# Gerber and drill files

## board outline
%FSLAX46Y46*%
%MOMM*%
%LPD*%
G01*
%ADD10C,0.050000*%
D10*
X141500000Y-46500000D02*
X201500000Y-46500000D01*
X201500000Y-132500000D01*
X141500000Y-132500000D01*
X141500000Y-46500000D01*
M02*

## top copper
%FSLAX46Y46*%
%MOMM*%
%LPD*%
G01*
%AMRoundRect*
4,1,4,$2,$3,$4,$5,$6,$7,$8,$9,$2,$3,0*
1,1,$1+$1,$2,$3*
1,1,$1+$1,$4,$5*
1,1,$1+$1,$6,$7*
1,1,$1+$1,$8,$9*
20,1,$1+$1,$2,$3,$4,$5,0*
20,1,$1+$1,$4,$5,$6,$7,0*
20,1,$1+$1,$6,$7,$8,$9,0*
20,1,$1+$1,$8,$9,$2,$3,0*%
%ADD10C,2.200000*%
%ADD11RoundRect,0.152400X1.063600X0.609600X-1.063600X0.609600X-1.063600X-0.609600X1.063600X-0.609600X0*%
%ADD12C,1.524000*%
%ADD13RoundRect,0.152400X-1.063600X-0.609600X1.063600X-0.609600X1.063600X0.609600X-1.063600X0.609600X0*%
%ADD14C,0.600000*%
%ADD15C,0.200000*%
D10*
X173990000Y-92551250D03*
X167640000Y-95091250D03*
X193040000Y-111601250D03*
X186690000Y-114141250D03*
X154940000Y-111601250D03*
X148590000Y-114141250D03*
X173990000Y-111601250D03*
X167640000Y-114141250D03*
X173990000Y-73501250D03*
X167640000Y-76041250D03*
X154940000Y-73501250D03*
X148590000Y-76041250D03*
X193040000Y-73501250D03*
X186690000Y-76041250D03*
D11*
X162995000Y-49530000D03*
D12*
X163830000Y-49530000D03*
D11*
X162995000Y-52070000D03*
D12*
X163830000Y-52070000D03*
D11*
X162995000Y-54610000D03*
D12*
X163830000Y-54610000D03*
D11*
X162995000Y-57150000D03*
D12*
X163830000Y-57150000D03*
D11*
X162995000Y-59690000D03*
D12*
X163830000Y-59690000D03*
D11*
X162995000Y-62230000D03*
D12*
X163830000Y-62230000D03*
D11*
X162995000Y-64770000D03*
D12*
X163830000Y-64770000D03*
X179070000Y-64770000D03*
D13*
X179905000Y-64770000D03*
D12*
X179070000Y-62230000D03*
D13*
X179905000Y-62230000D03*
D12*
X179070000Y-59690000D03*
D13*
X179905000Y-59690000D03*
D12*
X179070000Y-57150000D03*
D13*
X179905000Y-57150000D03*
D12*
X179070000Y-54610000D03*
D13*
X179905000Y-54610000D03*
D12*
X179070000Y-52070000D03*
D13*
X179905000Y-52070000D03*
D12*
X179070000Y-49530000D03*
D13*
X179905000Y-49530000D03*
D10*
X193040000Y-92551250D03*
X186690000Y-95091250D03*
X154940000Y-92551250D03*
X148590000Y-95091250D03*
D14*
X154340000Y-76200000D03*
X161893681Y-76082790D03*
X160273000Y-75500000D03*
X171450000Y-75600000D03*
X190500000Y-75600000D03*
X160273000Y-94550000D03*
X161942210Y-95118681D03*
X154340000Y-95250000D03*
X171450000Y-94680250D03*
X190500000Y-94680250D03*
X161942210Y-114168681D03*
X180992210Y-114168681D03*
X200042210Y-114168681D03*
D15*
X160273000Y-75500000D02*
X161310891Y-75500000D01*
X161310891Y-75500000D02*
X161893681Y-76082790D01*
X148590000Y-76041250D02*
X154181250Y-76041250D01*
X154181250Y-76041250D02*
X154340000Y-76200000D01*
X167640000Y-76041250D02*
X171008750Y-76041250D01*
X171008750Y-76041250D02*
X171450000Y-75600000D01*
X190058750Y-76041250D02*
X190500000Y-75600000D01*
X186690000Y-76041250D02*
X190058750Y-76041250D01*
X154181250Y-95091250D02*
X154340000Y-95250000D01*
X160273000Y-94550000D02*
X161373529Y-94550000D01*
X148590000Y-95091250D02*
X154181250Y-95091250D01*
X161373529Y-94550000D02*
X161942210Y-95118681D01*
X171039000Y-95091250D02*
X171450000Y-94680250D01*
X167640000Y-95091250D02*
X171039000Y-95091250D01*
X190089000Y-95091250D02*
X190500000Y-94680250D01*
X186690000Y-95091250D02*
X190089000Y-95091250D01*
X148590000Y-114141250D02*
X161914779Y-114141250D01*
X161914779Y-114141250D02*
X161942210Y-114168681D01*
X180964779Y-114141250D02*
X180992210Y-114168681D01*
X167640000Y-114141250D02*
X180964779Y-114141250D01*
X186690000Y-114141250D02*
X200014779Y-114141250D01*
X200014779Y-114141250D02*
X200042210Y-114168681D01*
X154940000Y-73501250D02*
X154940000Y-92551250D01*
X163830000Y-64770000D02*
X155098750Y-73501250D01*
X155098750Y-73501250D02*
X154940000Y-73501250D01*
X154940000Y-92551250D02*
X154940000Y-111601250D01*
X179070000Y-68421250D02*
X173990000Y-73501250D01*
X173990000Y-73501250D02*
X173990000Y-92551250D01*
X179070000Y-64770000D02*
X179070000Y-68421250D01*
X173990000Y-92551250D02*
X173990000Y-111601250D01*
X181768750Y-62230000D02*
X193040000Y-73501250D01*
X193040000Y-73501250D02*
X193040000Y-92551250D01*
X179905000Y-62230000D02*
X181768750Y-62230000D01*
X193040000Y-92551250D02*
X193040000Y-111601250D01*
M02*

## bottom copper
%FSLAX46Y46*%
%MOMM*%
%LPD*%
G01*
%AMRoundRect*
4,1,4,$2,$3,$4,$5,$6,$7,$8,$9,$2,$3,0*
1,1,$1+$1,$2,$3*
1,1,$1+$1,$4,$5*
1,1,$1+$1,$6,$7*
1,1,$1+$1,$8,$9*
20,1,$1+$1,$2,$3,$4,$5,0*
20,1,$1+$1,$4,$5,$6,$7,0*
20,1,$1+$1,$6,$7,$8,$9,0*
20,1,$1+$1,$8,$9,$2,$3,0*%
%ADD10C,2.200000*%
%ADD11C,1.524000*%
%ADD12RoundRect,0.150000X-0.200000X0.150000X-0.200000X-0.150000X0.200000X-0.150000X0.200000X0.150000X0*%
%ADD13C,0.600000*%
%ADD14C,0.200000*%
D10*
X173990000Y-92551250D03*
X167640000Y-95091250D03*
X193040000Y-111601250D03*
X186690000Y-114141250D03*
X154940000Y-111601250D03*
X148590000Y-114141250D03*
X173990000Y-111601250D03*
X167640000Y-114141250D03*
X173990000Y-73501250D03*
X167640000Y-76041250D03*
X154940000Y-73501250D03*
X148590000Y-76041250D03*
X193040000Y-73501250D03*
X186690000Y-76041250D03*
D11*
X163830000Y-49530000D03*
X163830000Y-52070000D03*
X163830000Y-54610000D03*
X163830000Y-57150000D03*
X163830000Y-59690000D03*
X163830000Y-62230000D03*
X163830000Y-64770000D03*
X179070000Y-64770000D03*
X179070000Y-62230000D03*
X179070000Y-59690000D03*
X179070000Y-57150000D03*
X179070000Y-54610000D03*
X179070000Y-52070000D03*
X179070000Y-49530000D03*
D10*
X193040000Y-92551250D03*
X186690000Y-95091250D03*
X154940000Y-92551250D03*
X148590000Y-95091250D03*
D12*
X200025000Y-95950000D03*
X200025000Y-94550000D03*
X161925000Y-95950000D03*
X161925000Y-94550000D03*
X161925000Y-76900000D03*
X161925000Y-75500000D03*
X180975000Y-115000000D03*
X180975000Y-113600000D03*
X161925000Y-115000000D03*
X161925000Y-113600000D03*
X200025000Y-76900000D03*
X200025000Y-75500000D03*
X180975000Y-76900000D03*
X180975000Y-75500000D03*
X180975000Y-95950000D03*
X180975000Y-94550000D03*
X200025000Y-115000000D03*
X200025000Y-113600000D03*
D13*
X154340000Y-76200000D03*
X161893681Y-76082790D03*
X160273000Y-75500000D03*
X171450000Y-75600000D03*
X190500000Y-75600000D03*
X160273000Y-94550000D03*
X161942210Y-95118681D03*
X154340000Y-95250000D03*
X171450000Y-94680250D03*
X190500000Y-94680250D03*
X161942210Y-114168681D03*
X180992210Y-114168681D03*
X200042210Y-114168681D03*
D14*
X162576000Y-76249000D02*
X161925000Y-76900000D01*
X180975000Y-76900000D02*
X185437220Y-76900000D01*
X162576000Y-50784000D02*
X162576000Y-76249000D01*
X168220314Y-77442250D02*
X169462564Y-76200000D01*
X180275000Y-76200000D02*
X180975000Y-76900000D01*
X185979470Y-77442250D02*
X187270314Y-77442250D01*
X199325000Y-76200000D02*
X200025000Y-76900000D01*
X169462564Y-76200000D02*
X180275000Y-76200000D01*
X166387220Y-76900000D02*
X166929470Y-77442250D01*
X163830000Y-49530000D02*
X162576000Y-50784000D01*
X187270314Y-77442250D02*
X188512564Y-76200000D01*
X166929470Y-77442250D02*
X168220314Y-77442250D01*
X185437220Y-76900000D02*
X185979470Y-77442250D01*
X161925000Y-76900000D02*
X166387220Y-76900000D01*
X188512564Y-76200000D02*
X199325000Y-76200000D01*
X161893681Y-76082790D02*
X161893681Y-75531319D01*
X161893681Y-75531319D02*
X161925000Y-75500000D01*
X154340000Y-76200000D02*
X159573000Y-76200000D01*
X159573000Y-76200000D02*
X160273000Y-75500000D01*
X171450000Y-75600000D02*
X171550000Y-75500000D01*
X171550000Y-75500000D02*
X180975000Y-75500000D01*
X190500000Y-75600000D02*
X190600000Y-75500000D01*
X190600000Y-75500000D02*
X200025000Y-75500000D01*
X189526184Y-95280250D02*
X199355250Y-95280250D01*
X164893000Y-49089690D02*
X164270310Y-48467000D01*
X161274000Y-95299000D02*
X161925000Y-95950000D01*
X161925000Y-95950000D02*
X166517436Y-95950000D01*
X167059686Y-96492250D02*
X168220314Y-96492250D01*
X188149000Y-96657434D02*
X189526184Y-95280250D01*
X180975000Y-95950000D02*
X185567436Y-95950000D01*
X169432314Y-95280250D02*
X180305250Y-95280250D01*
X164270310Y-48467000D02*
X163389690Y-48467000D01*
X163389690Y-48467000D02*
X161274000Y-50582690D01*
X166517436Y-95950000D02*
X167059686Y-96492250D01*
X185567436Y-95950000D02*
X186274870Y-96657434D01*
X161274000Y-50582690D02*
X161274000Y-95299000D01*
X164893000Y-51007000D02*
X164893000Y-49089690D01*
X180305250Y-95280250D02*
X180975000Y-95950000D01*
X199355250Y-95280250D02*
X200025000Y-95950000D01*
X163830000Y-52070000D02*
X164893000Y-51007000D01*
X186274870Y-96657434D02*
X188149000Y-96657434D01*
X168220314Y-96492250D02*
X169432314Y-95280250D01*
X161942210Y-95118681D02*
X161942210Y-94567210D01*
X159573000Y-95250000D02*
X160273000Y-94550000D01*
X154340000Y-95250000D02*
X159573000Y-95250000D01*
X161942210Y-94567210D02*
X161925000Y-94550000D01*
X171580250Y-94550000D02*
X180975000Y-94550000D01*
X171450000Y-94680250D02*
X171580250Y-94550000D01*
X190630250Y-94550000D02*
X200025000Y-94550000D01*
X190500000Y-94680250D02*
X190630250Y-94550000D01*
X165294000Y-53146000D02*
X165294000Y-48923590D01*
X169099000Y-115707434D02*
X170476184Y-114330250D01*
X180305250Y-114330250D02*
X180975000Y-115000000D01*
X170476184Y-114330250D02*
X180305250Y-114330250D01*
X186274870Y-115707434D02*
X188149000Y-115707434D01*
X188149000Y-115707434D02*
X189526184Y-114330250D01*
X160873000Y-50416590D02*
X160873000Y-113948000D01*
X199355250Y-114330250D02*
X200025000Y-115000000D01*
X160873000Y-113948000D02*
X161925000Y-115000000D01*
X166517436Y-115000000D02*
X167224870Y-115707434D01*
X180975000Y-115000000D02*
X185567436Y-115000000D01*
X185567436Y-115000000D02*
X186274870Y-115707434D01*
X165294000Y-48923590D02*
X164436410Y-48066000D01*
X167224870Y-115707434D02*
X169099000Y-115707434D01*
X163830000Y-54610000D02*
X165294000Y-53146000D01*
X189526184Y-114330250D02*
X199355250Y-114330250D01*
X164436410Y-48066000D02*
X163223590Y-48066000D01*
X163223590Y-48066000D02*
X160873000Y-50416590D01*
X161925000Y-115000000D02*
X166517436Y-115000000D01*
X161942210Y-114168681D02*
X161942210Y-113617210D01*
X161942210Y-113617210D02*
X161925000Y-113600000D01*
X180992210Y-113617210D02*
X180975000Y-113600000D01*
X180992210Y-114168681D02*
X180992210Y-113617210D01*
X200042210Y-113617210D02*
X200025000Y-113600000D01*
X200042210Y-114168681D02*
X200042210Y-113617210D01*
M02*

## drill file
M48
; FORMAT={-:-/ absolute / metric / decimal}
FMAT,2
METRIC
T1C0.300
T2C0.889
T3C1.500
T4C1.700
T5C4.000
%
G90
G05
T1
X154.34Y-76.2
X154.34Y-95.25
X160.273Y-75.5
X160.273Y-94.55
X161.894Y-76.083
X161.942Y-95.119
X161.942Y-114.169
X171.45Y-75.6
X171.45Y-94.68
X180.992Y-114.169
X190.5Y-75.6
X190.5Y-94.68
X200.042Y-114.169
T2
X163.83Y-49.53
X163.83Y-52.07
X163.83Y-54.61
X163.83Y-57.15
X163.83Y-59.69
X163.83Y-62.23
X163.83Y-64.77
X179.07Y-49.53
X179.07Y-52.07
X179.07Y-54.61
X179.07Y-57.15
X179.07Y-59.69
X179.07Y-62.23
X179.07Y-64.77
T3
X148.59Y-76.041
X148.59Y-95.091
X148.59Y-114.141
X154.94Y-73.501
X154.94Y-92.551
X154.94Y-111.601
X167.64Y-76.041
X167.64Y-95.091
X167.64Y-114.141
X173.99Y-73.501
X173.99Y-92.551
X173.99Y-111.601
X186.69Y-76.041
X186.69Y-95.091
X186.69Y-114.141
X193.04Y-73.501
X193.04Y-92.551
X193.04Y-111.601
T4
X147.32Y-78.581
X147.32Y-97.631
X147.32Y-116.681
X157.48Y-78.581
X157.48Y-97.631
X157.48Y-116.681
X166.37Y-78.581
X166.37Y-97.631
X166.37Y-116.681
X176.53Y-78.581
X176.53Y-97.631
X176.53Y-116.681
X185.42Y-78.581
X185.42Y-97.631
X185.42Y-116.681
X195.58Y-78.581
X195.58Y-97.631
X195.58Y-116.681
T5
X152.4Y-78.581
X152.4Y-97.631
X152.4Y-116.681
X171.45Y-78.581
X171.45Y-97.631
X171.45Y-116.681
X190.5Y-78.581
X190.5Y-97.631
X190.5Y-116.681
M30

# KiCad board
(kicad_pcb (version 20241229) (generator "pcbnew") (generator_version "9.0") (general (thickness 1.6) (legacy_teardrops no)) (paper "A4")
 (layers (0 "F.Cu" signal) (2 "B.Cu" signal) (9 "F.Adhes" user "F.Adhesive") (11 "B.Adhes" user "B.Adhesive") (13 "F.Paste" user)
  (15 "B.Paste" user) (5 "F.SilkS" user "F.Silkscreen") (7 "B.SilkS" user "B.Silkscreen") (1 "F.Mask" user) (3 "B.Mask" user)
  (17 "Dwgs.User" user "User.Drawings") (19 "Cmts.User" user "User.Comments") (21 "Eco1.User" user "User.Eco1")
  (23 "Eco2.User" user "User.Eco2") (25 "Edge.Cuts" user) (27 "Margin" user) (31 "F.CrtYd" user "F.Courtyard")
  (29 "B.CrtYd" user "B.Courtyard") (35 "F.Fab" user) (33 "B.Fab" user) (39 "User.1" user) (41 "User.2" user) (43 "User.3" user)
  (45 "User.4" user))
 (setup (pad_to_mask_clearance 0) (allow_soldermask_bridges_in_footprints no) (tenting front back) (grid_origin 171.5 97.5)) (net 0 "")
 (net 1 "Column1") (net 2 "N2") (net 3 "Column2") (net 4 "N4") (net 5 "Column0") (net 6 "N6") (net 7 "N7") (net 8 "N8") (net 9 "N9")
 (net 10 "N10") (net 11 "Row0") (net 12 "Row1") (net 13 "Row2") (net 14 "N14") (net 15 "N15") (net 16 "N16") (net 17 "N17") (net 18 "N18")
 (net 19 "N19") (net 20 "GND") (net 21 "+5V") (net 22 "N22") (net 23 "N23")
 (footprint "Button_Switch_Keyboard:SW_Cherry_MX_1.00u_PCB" (layer "F.Cu") (at 173.99 92.55125)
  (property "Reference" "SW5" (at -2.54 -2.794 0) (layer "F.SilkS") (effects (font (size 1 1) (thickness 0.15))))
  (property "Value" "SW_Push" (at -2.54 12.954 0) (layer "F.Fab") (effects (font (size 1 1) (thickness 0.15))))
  (pad "" np_thru_hole circle (at -7.62 5.08) (size 1.7 1.7) (drill 1.7) (layers "*.Cu" "*.Mask"))
  (pad "" np_thru_hole circle (at -2.54 5.08) (size 4 4) (drill 4) (layers "*.Cu" "*.Mask"))
  (pad "" np_thru_hole circle (at 2.54 5.08) (size 1.7 1.7) (drill 1.7) (layers "*.Cu" "*.Mask"))
  (pad "1" thru_hole circle (at 0 0) (size 2.2 2.2) (drill 1.5) (layers "*.Cu" "*.Mask") (remove_unused_layers no) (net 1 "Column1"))
  (pad "2" thru_hole circle (at -6.35 2.54) (size 2.2 2.2) (drill 1.5) (layers "*.Cu" "*.Mask") (remove_unused_layers no) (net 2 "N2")))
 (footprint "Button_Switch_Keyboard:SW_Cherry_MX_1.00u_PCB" (layer "F.Cu") (at 193.04 111.60125)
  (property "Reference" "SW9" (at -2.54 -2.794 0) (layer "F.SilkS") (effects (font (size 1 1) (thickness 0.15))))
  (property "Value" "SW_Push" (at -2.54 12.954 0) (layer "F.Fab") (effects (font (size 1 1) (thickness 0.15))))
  (pad "" np_thru_hole circle (at -7.62 5.08) (size 1.7 1.7) (drill 1.7) (layers "*.Cu" "*.Mask"))
  (pad "" np_thru_hole circle (at -2.54 5.08) (size 4 4) (drill 4) (layers "*.Cu" "*.Mask"))
  (pad "" np_thru_hole circle (at 2.54 5.08) (size 1.7 1.7) (drill 1.7) (layers "*.Cu" "*.Mask"))
  (pad "1" thru_hole circle (at 0 0) (size 2.2 2.2) (drill 1.5) (layers "*.Cu" "*.Mask") (remove_unused_layers no) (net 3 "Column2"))
  (pad "2" thru_hole circle (at -6.35 2.54) (size 2.2 2.2) (drill 1.5) (layers "*.Cu" "*.Mask") (remove_unused_layers no) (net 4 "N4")))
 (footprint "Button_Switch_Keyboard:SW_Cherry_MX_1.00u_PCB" (layer "F.Cu") (at 154.94 111.60125)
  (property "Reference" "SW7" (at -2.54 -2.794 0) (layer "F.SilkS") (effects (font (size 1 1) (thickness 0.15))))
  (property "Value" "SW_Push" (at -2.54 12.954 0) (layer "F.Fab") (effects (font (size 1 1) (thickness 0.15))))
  (pad "" np_thru_hole circle (at -7.62 5.08) (size 1.7 1.7) (drill 1.7) (layers "*.Cu" "*.Mask"))
  (pad "" np_thru_hole circle (at -2.54 5.08) (size 4 4) (drill 4) (layers "*.Cu" "*.Mask"))
  (pad "" np_thru_hole circle (at 2.54 5.08) (size 1.7 1.7) (drill 1.7) (layers "*.Cu" "*.Mask"))
  (pad "1" thru_hole circle (at 0 0) (size 2.2 2.2) (drill 1.5) (layers "*.Cu" "*.Mask") (remove_unused_layers no) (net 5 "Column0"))
  (pad "2" thru_hole circle (at -6.35 2.54) (size 2.2 2.2) (drill 1.5) (layers "*.Cu" "*.Mask") (remove_unused_layers no) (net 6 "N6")))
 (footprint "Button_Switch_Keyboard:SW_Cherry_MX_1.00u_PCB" (layer "F.Cu") (at 173.99 111.60125)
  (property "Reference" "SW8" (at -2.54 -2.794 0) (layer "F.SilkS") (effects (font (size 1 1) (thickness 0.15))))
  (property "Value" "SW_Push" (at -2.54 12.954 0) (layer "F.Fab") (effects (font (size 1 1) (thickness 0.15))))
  (pad "" np_thru_hole circle (at -7.62 5.08) (size 1.7 1.7) (drill 1.7) (layers "*.Cu" "*.Mask"))
  (pad "" np_thru_hole circle (at -2.54 5.08) (size 4 4) (drill 4) (layers "*.Cu" "*.Mask"))
  (pad "" np_thru_hole circle (at 2.54 5.08) (size 1.7 1.7) (drill 1.7) (layers "*.Cu" "*.Mask"))
  (pad "1" thru_hole circle (at 0 0) (size 2.2 2.2) (drill 1.5) (layers "*.Cu" "*.Mask") (remove_unused_layers no) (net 1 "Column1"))
  (pad "2" thru_hole circle (at -6.35 2.54) (size 2.2 2.2) (drill 1.5) (layers "*.Cu" "*.Mask") (remove_unused_layers no) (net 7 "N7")))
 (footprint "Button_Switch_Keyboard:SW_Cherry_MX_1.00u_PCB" (layer "F.Cu") (at 173.99 73.50125)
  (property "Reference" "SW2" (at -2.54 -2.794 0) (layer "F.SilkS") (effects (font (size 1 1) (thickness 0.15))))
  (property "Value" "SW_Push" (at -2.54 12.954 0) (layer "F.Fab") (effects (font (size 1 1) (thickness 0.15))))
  (pad "" np_thru_hole circle (at -7.62 5.08) (size 1.7 1.7) (drill 1.7) (layers "*.Cu" "*.Mask"))
  (pad "" np_thru_hole circle (at -2.54 5.08) (size 4 4) (drill 4) (layers "*.Cu" "*.Mask"))
  (pad "" np_thru_hole circle (at 2.54 5.08) (size 1.7 1.7) (drill 1.7) (layers "*.Cu" "*.Mask"))
  (pad "1" thru_hole circle (at 0 0) (size 2.2 2.2) (drill 1.5) (layers "*.Cu" "*.Mask") (remove_unused_layers no) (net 1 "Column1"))
  (pad "2" thru_hole circle (at -6.35 2.54) (size 2.2 2.2) (drill 1.5) (layers "*.Cu" "*.Mask") (remove_unused_layers no) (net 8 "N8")))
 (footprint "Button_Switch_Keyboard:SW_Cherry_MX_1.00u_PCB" (layer "F.Cu") (at 154.94 73.50125)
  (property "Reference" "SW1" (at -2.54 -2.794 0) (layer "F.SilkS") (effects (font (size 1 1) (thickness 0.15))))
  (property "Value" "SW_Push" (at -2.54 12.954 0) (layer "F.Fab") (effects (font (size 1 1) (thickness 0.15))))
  (pad "" np_thru_hole circle (at -7.62 5.08) (size 1.7 1.7) (drill 1.7) (layers "*.Cu" "*.Mask"))
  (pad "" np_thru_hole circle (at -2.54 5.08) (size 4 4) (drill 4) (layers "*.Cu" "*.Mask"))
  (pad "" np_thru_hole circle (at 2.54 5.08) (size 1.7 1.7) (drill 1.7) (layers "*.Cu" "*.Mask"))
  (pad "1" thru_hole circle (at 0 0) (size 2.2 2.2) (drill 1.5) (layers "*.Cu" "*.Mask") (remove_unused_layers no) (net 5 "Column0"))
  (pad "2" thru_hole circle (at -6.35 2.54) (size 2.2 2.2) (drill 1.5) (layers "*.Cu" "*.Mask") (remove_unused_layers no) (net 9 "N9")))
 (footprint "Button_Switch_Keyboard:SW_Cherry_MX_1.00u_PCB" (layer "F.Cu") (at 193.04 73.50125)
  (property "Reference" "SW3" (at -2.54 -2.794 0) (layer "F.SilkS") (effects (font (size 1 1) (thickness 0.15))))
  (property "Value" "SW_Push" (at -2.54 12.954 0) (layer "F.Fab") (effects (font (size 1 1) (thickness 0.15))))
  (pad "" np_thru_hole circle (at -7.62 5.08) (size 1.7 1.7) (drill 1.7) (layers "*.Cu" "*.Mask"))
  (pad "" np_thru_hole circle (at -2.54 5.08) (size 4 4) (drill 4) (layers "*.Cu" "*.Mask"))
  (pad "" np_thru_hole circle (at 2.54 5.08) (size 1.7 1.7) (drill 1.7) (layers "*.Cu" "*.Mask"))
  (pad "1" thru_hole circle (at 0 0) (size 2.2 2.2) (drill 1.5) (layers "*.Cu" "*.Mask") (remove_unused_layers no) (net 3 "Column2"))
  (pad "2" thru_hole circle (at -6.35 2.54) (size 2.2 2.2) (drill 1.5) (layers "*.Cu" "*.Mask") (remove_unused_layers no) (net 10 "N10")))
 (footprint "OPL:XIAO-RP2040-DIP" (layer "F.Cu") (at 171.45 57.15)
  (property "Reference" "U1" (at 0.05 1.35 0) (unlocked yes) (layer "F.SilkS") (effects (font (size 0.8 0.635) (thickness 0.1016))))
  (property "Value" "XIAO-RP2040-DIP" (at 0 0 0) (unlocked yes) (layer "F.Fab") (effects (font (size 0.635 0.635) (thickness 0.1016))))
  (pad "1" smd roundrect (at -8.455 -7.62 180) (size 2.432 1.524) (layers "F.Cu" "F.Mask") (roundrect_rratio 0.1) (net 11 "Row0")
   (thermal_bridge_angle 45))
  (pad "1" thru_hole circle (at -7.62 -7.62 180) (size 1.524 1.524) (drill 0.889) (layers "*.Cu" "*.Mask") (remove_unused_layers no)
   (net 11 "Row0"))
  (pad "2" smd roundrect (at -8.455 -5.08 180) (size 2.432 1.524) (layers "F.Cu" "F.Mask") (roundrect_rratio 0.1) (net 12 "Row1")
   (thermal_bridge_angle 45))
  (pad "2" thru_hole circle (at -7.62 -5.08 180) (size 1.524 1.524) (drill 0.889) (layers "*.Cu" "*.Mask") (remove_unused_layers no)
   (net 12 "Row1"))
  (pad "3" smd roundrect (at -8.455 -2.54 180) (size 2.432 1.524) (layers "F.Cu" "F.Mask") (roundrect_rratio 0.1) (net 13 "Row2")
   (thermal_bridge_angle 45))
  (pad "3" thru_hole circle (at -7.62 -2.54 180) (size 1.524 1.524) (drill 0.889) (layers "*.Cu" "*.Mask") (remove_unused_layers no)
   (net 13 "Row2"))
  (pad "4" smd roundrect (at -8.455 0 180) (size 2.432 1.524) (layers "F.Cu" "F.Mask") (roundrect_rratio 0.1) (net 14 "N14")
   (thermal_bridge_angle 45))
  (pad "4" thru_hole circle (at -7.62 0 180) (size 1.524 1.524) (drill 0.889) (layers "*.Cu" "*.Mask") (remove_unused_layers no)
   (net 14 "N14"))
  (pad "5" smd roundrect (at -8.455 2.54 180) (size 2.432 1.524) (layers "F.Cu" "F.Mask") (roundrect_rratio 0.1) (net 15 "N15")
   (thermal_bridge_angle 45))
  (pad "5" thru_hole circle (at -7.62 2.54 180) (size 1.524 1.524) (drill 0.889) (layers "*.Cu" "*.Mask") (remove_unused_layers no)
   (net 15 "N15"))
  (pad "6" smd roundrect (at -8.455 5.08 180) (size 2.432 1.524) (layers "F.Cu" "F.Mask") (roundrect_rratio 0.1) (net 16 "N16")
   (thermal_bridge_angle 45))
  (pad "6" thru_hole circle (at -7.62 5.08 180) (size 1.524 1.524) (drill 0.889) (layers "*.Cu" "*.Mask") (remove_unused_layers no)
   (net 16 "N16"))
  (pad "7" smd roundrect (at -8.455 7.62 180) (size 2.432 1.524) (layers "F.Cu" "F.Mask") (roundrect_rratio 0.1) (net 5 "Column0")
   (thermal_bridge_angle 45))
  (pad "7" thru_hole circle (at -7.62 7.62 180) (size 1.524 1.524) (drill 0.889) (layers "*.Cu" "*.Mask") (remove_unused_layers no)
   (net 5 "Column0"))
  (pad "8" thru_hole circle (at 7.62 7.62) (size 1.524 1.524) (drill 0.889) (layers "*.Cu" "*.Mask") (remove_unused_layers no)
   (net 1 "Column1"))
  (pad "8" smd roundrect (at 8.455 7.62) (size 2.432 1.524) (layers "F.Cu" "F.Mask") (roundrect_rratio 0.1) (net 1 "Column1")
   (thermal_bridge_angle 45))
  (pad "9" thru_hole circle (at 7.62 5.08) (size 1.524 1.524) (drill 0.889) (layers "*.Cu" "*.Mask") (remove_unused_layers no)
   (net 3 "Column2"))
  (pad "9" smd roundrect (at 8.455 5.08) (size 2.432 1.524) (layers "F.Cu" "F.Mask") (roundrect_rratio 0.1) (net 3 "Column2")
   (thermal_bridge_angle 45))
  (pad "10" thru_hole circle (at 7.62 2.54) (size 1.524 1.524) (drill 0.889) (layers "*.Cu" "*.Mask") (remove_unused_layers no)
   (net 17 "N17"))
  (pad "10" smd roundrect (at 8.455 2.54) (size 2.432 1.524) (layers "F.Cu" "F.Mask") (roundrect_rratio 0.1) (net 17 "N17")
   (thermal_bridge_angle 45))
  (pad "11" thru_hole circle (at 7.62 0) (size 1.524 1.524) (drill 0.889) (layers "*.Cu" "*.Mask") (remove_unused_layers no) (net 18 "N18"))
  (pad "11" smd roundrect (at 8.455 0) (size 2.432 1.524) (layers "F.Cu" "F.Mask") (roundrect_rratio 0.1) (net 18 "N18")
   (thermal_bridge_angle 45))
  (pad "12" thru_hole circle (at 7.62 -2.54) (size 1.524 1.524) (drill 0.889) (layers "*.Cu" "*.Mask") (remove_unused_layers no)
   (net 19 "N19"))
  (pad "12" smd roundrect (at 8.455 -2.54) (size 2.432 1.524) (layers "F.Cu" "F.Mask") (roundrect_rratio 0.1) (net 19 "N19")
   (thermal_bridge_angle 45))
  (pad "13" thru_hole circle (at 7.62 -5.08) (size 1.524 1.524) (drill 0.889) (layers "*.Cu" "*.Mask") (remove_unused_layers no)
   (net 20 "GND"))
  (pad "13" smd roundrect (at 8.455 -5.08) (size 2.432 1.524) (layers "F.Cu" "F.Mask") (roundrect_rratio 0.1) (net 20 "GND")
   (thermal_bridge_angle 45))
  (pad "14" thru_hole circle (at 7.62 -7.62) (size 1.524 1.524) (drill 0.889) (layers "*.Cu" "*.Mask") (remove_unused_layers no)
   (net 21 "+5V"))
  (pad "14" smd roundrect (at 8.455 -7.62) (size 2.432 1.524) (layers "F.Cu" "F.Mask") (roundrect_rratio 0.1) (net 21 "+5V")
   (thermal_bridge_angle 45)))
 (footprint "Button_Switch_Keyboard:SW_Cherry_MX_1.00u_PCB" (layer "F.Cu") (at 193.04 92.55125)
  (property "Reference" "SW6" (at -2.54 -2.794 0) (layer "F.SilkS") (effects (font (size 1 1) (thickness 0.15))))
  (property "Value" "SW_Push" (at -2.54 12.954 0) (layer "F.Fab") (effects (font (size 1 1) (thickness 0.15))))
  (pad "" np_thru_hole circle (at -7.62 5.08) (size 1.7 1.7) (drill 1.7) (layers "*.Cu" "*.Mask"))
  (pad "" np_thru_hole circle (at -2.54 5.08) (size 4 4) (drill 4) (layers "*.Cu" "*.Mask"))
  (pad "" np_thru_hole circle (at 2.54 5.08) (size 1.7 1.7) (drill 1.7) (layers "*.Cu" "*.Mask"))
  (pad "1" thru_hole circle (at 0 0) (size 2.2 2.2) (drill 1.5) (layers "*.Cu" "*.Mask") (remove_unused_layers no) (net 3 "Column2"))
  (pad "2" thru_hole circle (at -6.35 2.54) (size 2.2 2.2) (drill 1.5) (layers "*.Cu" "*.Mask") (remove_unused_layers no) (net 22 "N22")))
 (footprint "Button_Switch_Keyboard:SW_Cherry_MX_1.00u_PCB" (layer "F.Cu") (at 154.94 92.55125)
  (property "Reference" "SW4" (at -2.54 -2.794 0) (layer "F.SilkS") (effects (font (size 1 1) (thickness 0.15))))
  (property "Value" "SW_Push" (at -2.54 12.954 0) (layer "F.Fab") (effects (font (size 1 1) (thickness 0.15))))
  (pad "" np_thru_hole circle (at -7.62 5.08) (size 1.7 1.7) (drill 1.7) (layers "*.Cu" "*.Mask"))
  (pad "" np_thru_hole circle (at -2.54 5.08) (size 4 4) (drill 4) (layers "*.Cu" "*.Mask"))
  (pad "" np_thru_hole circle (at 2.54 5.08) (size 1.7 1.7) (drill 1.7) (layers "*.Cu" "*.Mask"))
  (pad "1" thru_hole circle (at 0 0) (size 2.2 2.2) (drill 1.5) (layers "*.Cu" "*.Mask") (remove_unused_layers no) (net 5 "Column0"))
  (pad "2" thru_hole circle (at -6.35 2.54) (size 2.2 2.2) (drill 1.5) (layers "*.Cu" "*.Mask") (remove_unused_layers no) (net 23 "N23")))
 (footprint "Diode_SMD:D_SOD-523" (layer "B.Cu") (at 200.025 95.25 90)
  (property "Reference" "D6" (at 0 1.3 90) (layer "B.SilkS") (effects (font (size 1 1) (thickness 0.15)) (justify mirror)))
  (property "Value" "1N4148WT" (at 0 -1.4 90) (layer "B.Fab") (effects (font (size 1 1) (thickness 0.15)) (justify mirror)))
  (pad "1" smd roundrect (at -0.7 0 270) (size 0.6 0.7) (layers "B.Cu" "B.Mask" "B.Paste") (roundrect_rratio 0.25) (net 12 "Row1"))
  (pad "2" smd roundrect (at 0.7 0 270) (size 0.6 0.7) (layers "B.Cu" "B.Mask" "B.Paste") (roundrect_rratio 0.25) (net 22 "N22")))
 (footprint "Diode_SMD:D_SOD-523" (layer "B.Cu") (at 161.925 95.25 90)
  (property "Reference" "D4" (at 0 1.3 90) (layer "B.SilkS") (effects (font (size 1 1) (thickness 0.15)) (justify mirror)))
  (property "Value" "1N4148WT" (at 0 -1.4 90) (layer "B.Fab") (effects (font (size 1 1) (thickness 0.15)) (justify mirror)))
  (pad "1" smd roundrect (at -0.7 0 270) (size 0.6 0.7) (layers "B.Cu" "B.Mask" "B.Paste") (roundrect_rratio 0.25) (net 12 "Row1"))
  (pad "2" smd roundrect (at 0.7 0 270) (size 0.6 0.7) (layers "B.Cu" "B.Mask" "B.Paste") (roundrect_rratio 0.25) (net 23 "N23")))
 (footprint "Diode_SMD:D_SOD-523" (layer "B.Cu") (at 161.925 76.2 90)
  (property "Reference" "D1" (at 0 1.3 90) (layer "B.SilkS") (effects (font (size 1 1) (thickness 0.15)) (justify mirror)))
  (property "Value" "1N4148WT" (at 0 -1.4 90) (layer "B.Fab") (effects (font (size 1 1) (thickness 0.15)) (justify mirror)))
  (pad "1" smd roundrect (at -0.7 0 270) (size 0.6 0.7) (layers "B.Cu" "B.Mask" "B.Paste") (roundrect_rratio 0.25) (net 11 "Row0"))
  (pad "2" smd roundrect (at 0.7 0 270) (size 0.6 0.7) (layers "B.Cu" "B.Mask" "B.Paste") (roundrect_rratio 0.25) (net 9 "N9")))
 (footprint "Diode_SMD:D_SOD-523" (layer "B.Cu") (at 180.975 114.3 90)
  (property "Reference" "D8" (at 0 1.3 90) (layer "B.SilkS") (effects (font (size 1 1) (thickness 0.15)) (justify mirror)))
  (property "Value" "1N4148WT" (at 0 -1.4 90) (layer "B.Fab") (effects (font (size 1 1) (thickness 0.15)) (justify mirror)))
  (pad "1" smd roundrect (at -0.7 0 270) (size 0.6 0.7) (layers "B.Cu" "B.Mask" "B.Paste") (roundrect_rratio 0.25) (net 13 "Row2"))
  (pad "2" smd roundrect (at 0.7 0 270) (size 0.6 0.7) (layers "B.Cu" "B.Mask" "B.Paste") (roundrect_rratio 0.25) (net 7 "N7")))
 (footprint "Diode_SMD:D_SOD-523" (layer "B.Cu") (at 161.925 114.3 90)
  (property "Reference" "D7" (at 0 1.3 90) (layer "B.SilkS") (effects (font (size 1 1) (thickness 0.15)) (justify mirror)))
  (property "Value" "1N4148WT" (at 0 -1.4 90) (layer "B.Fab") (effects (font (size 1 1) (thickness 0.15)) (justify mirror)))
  (pad "1" smd roundrect (at -0.7 0 270) (size 0.6 0.7) (layers "B.Cu" "B.Mask" "B.Paste") (roundrect_rratio 0.25) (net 13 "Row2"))
  (pad "2" smd roundrect (at 0.7 0 270) (size 0.6 0.7) (layers "B.Cu" "B.Mask" "B.Paste") (roundrect_rratio 0.25) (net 6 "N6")))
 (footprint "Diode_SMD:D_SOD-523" (layer "B.Cu") (at 200.025 76.2 90)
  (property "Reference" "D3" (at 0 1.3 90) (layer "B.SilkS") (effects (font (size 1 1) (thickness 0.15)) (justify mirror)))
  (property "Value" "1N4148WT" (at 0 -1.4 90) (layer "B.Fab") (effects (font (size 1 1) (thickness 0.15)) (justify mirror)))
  (pad "1" smd roundrect (at -0.7 0 270) (size 0.6 0.7) (layers "B.Cu" "B.Mask" "B.Paste") (roundrect_rratio 0.25) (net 11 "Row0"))
  (pad "2" smd roundrect (at 0.7 0 270) (size 0.6 0.7) (layers "B.Cu" "B.Mask" "B.Paste") (roundrect_rratio 0.25) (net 10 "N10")))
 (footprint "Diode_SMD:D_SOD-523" (layer "B.Cu") (at 180.975 76.2 90)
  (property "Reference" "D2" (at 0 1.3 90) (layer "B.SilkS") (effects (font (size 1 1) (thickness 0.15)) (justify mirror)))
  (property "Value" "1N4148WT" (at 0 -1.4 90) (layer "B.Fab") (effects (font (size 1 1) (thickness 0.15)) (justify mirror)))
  (pad "1" smd roundrect (at -0.7 0 270) (size 0.6 0.7) (layers "B.Cu" "B.Mask" "B.Paste") (roundrect_rratio 0.25) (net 11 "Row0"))
  (pad "2" smd roundrect (at 0.7 0 270) (size 0.6 0.7) (layers "B.Cu" "B.Mask" "B.Paste") (roundrect_rratio 0.25) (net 8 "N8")))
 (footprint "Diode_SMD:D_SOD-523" (layer "B.Cu") (at 180.975 95.25 90)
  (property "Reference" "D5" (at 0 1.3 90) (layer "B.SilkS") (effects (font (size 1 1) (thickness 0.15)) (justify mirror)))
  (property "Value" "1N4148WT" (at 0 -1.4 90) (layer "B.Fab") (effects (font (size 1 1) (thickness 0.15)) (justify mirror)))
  (pad "1" smd roundrect (at -0.7 0 270) (size 0.6 0.7) (layers "B.Cu" "B.Mask" "B.Paste") (roundrect_rratio 0.25) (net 12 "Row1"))
  (pad "2" smd roundrect (at 0.7 0 270) (size 0.6 0.7) (layers "B.Cu" "B.Mask" "B.Paste") (roundrect_rratio 0.25) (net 2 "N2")))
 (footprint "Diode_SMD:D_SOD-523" (layer "B.Cu") (at 200.025 114.3 90)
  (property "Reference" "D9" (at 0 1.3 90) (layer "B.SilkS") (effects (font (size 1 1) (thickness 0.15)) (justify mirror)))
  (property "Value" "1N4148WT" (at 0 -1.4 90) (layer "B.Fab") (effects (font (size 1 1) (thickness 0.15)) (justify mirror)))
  (pad "1" smd roundrect (at -0.7 0 270) (size 0.6 0.7) (layers "B.Cu" "B.Mask" "B.Paste") (roundrect_rratio 0.25) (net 13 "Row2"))
  (pad "2" smd roundrect (at 0.7 0 270) (size 0.6 0.7) (layers "B.Cu" "B.Mask" "B.Paste") (roundrect_rratio 0.25) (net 4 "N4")))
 (gr_rect (start 141.5 46.5) (end 201.5 132.5) (stroke (width 0.05) (type default)) (fill no) (layer "Edge.Cuts"))
 (segment (start 162.576 76.249) (end 161.925 76.9) (width 0.2) (layer "B.Cu") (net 11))
 (segment (start 180.975 76.9) (end 185.43722 76.9) (width 0.2) (layer "B.Cu") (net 11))
 (segment (start 162.576 50.784) (end 162.576 76.249) (width 0.2) (layer "B.Cu") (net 11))
 (segment (start 168.220314 77.44225) (end 169.462564 76.2) (width 0.2) (layer "B.Cu") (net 11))
 (segment (start 180.275 76.2) (end 180.975 76.9) (width 0.2) (layer "B.Cu") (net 11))
 (segment (start 185.97947 77.44225) (end 187.270314 77.44225) (width 0.2) (layer "B.Cu") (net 11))
 (segment (start 199.325 76.2) (end 200.025 76.9) (width 0.2) (layer "B.Cu") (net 11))
 (segment (start 169.462564 76.2) (end 180.275 76.2) (width 0.2) (layer "B.Cu") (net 11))
 (segment (start 166.38722 76.9) (end 166.92947 77.44225) (width 0.2) (layer "B.Cu") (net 11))
 (segment (start 163.83 49.53) (end 162.576 50.784) (width 0.2) (layer "B.Cu") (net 11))
 (segment (start 187.270314 77.44225) (end 188.512564 76.2) (width 0.2) (layer "B.Cu") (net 11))
 (segment (start 166.92947 77.44225) (end 168.220314 77.44225) (width 0.2) (layer "B.Cu") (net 11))
 (segment (start 185.43722 76.9) (end 185.97947 77.44225) (width 0.2) (layer "B.Cu") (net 11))
 (segment (start 161.925 76.9) (end 166.38722 76.9) (width 0.2) (layer "B.Cu") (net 11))
 (segment (start 188.512564 76.2) (end 199.325 76.2) (width 0.2) (layer "B.Cu") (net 11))
 (segment (start 160.273 75.5) (end 161.310891 75.5) (width 0.2) (layer "F.Cu") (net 9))
 (segment (start 161.310891 75.5) (end 161.893681 76.08279) (width 0.2) (layer "F.Cu") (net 9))
 (segment (start 148.59 76.04125) (end 154.18125 76.04125) (width 0.2) (layer "F.Cu") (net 9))
 (segment (start 154.18125 76.04125) (end 154.34 76.2) (width 0.2) (layer "F.Cu") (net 9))
 (via (at 154.34 76.2) (size 0.6) (drill 0.3) (layers "F.Cu" "B.Cu") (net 9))
 (via (at 161.893681 76.08279) (size 0.6) (drill 0.3) (layers "F.Cu" "B.Cu") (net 9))
 (via (at 160.273 75.5) (size 0.6) (drill 0.3) (layers "F.Cu" "B.Cu") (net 9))
 (segment (start 161.893681 76.08279) (end 161.893681 75.531319) (width 0.2) (layer "B.Cu") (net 9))
 (segment (start 161.893681 75.531319) (end 161.925 75.5) (width 0.2) (layer "B.Cu") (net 9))
 (segment (start 154.34 76.2) (end 159.573 76.2) (width 0.2) (layer "B.Cu") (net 9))
 (segment (start 159.573 76.2) (end 160.273 75.5) (width 0.2) (layer "B.Cu") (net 9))
 (segment (start 167.64 76.04125) (end 171.00875 76.04125) (width 0.2) (layer "F.Cu") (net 8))
 (segment (start 171.00875 76.04125) (end 171.45 75.6) (width 0.2) (layer "F.Cu") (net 8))
 (via (at 171.45 75.6) (size 0.6) (drill 0.3) (layers "F.Cu" "B.Cu") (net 8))
 (segment (start 171.45 75.6) (end 171.55 75.5) (width 0.2) (layer "B.Cu") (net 8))
 (segment (start 171.55 75.5) (end 180.975 75.5) (width 0.2) (layer "B.Cu") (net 8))
 (segment (start 190.05875 76.04125) (end 190.5 75.6) (width 0.2) (layer "F.Cu") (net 10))
 (segment (start 186.69 76.04125) (end 190.05875 76.04125) (width 0.2) (layer "F.Cu") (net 10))
 (via (at 190.5 75.6) (size 0.6) (drill 0.3) (layers "F.Cu" "B.Cu") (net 10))
 (segment (start 190.5 75.6) (end 190.6 75.5) (width 0.2) (layer "B.Cu") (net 10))
 (segment (start 190.6 75.5) (end 200.025 75.5) (width 0.2) (layer "B.Cu") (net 10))
 (segment (start 189.526184 95.28025) (end 199.35525 95.28025) (width 0.2) (layer "B.Cu") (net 12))
 (segment (start 164.893 49.08969) (end 164.27031 48.467) (width 0.2) (layer "B.Cu") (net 12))
 (segment (start 161.274 95.299) (end 161.925 95.95) (width 0.2) (layer "B.Cu") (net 12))
 (segment (start 161.925 95.95) (end 166.517436 95.95) (width 0.2) (layer "B.Cu") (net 12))
 (segment (start 167.059686 96.49225) (end 168.220314 96.49225) (width 0.2) (layer "B.Cu") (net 12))
 (segment (start 188.149 96.657434) (end 189.526184 95.28025) (width 0.2) (layer "B.Cu") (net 12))
 (segment (start 180.975 95.95) (end 185.567436 95.95) (width 0.2) (layer "B.Cu") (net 12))
 (segment (start 169.432314 95.28025) (end 180.30525 95.28025) (width 0.2) (layer "B.Cu") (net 12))
 (segment (start 164.27031 48.467) (end 163.38969 48.467) (width 0.2) (layer "B.Cu") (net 12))
 (segment (start 163.38969 48.467) (end 161.274 50.58269) (width 0.2) (layer "B.Cu") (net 12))
 (segment (start 166.517436 95.95) (end 167.059686 96.49225) (width 0.2) (layer "B.Cu") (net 12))
 (segment (start 185.567436 95.95) (end 186.27487 96.657434) (width 0.2) (layer "B.Cu") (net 12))
 (segment (start 161.274 50.58269) (end 161.274 95.299) (width 0.2) (layer "B.Cu") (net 12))
 (segment (start 164.893 51.007) (end 164.893 49.08969) (width 0.2) (layer "B.Cu") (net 12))
 (segment (start 180.30525 95.28025) (end 180.975 95.95) (width 0.2) (layer "B.Cu") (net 12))
 (segment (start 199.35525 95.28025) (end 200.025 95.95) (width 0.2) (layer "B.Cu") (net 12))
 (segment (start 163.83 52.07) (end 164.893 51.007) (width 0.2) (layer "B.Cu") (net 12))
 (segment (start 186.27487 96.657434) (end 188.149 96.657434) (width 0.2) (layer "B.Cu") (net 12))
 (segment (start 168.220314 96.49225) (end 169.432314 95.28025) (width 0.2) (layer "B.Cu") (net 12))
 (segment (start 154.18125 95.09125) (end 154.34 95.25) (width 0.2) (layer "F.Cu") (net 23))
 (segment (start 160.273 94.55) (end 161.373529 94.55) (width 0.2) (layer "F.Cu") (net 23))
 (segment (start 148.59 95.09125) (end 154.18125 95.09125) (width 0.2) (layer "F.Cu") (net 23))
 (segment (start 161.373529 94.55) (end 161.94221 95.118681) (width 0.2) (layer "F.Cu") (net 23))
 (via (at 160.273 94.55) (size 0.6) (drill 0.3) (layers "F.Cu" "B.Cu") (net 23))
 (via (at 161.94221 95.118681) (size 0.6) (drill 0.3) (layers "F.Cu" "B.Cu") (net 23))
 (via (at 154.34 95.25) (size 0.6) (drill 0.3) (layers "F.Cu" "B.Cu") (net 23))
 (segment (start 161.94221 95.118681) (end 161.94221 94.56721) (width 0.2) (layer "B.Cu") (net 23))
 (segment (start 159.573 95.25) (end 160.273 94.55) (width 0.2) (layer "B.Cu") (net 23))
 (segment (start 154.34 95.25) (end 159.573 95.25) (width 0.2) (layer "B.Cu") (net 23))
 (segment (start 161.94221 94.56721) (end 161.925 94.55) (width 0.2) (layer "B.Cu") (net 23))
 (segment (start 171.039 95.09125) (end 171.45 94.68025) (width 0.2) (layer "F.Cu") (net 2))
 (segment (start 167.64 95.09125) (end 171.039 95.09125) (width 0.2) (layer "F.Cu") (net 2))
 (via (at 171.45 94.68025) (size 0.6) (drill 0.3) (layers "F.Cu" "B.Cu") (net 2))
 (segment (start 171.58025 94.55) (end 180.975 94.55) (width 0.2) (layer "B.Cu") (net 2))
 (segment (start 171.45 94.68025) (end 171.58025 94.55) (width 0.2) (layer "B.Cu") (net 2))
 (segment (start 190.089 95.09125) (end 190.5 94.68025) (width 0.2) (layer "F.Cu") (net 22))
 (segment (start 186.69 95.09125) (end 190.089 95.09125) (width 0.2) (layer "F.Cu") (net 22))
 (via (at 190.5 94.68025) (size 0.6) (drill 0.3) (layers "F.Cu" "B.Cu") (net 22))
 (segment (start 190.63025 94.55) (end 200.025 94.55) (width 0.2) (layer "B.Cu") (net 22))
 (segment (start 190.5 94.68025) (end 190.63025 94.55) (width 0.2) (layer "B.Cu") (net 22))
 (segment (start 165.294 53.146) (end 165.294 48.92359) (width 0.2) (layer "B.Cu") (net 13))
 (segment (start 169.099 115.707434) (end 170.476184 114.33025) (width 0.2) (layer "B.Cu") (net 13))
 (segment (start 180.30525 114.33025) (end 180.975 115) (width 0.2) (layer "B.Cu") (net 13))
 (segment (start 170.476184 114.33025) (end 180.30525 114.33025) (width 0.2) (layer "B.Cu") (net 13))
 (segment (start 186.27487 115.707434) (end 188.149 115.707434) (width 0.2) (layer "B.Cu") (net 13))
 (segment (start 188.149 115.707434) (end 189.526184 114.33025) (width 0.2) (layer "B.Cu") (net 13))
 (segment (start 160.873 50.41659) (end 160.873 113.948) (width 0.2) (layer "B.Cu") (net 13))
 (segment (start 199.35525 114.33025) (end 200.025 115) (width 0.2) (layer "B.Cu") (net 13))
 (segment (start 160.873 113.948) (end 161.925 115) (width 0.2) (layer "B.Cu") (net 13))
 (segment (start 166.517436 115) (end 167.22487 115.707434) (width 0.2) (layer "B.Cu") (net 13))
 (segment (start 180.975 115) (end 185.567436 115) (width 0.2) (layer "B.Cu") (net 13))
 (segment (start 185.567436 115) (end 186.27487 115.707434) (width 0.2) (layer "B.Cu") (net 13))
 (segment (start 165.294 48.92359) (end 164.43641 48.066) (width 0.2) (layer "B.Cu") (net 13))
 (segment (start 167.22487 115.707434) (end 169.099 115.707434) (width 0.2) (layer "B.Cu") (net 13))
 (segment (start 163.83 54.61) (end 165.294 53.146) (width 0.2) (layer "B.Cu") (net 13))
 (segment (start 189.526184 114.33025) (end 199.35525 114.33025) (width 0.2) (layer "B.Cu") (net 13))
 (segment (start 164.43641 48.066) (end 163.22359 48.066) (width 0.2) (layer "B.Cu") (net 13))
 (segment (start 163.22359 48.066) (end 160.873 50.41659) (width 0.2) (layer "B.Cu") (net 13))
 (segment (start 161.925 115) (end 166.517436 115) (width 0.2) (layer "B.Cu") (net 13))
 (segment (start 148.59 114.14125) (end 161.914779 114.14125) (width 0.2) (layer "F.Cu") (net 6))
 (segment (start 161.914779 114.14125) (end 161.94221 114.168681) (width 0.2) (layer "F.Cu") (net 6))
 (via (at 161.94221 114.168681) (size 0.6) (drill 0.3) (layers "F.Cu" "B.Cu") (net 6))
 (segment (start 161.94221 114.168681) (end 161.94221 113.61721) (width 0.2) (layer "B.Cu") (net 6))
 (segment (start 161.94221 113.61721) (end 161.925 113.6) (width 0.2) (layer "B.Cu") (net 6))
 (segment (start 180.964779 114.14125) (end 180.99221 114.168681) (width 0.2) (layer "F.Cu") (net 7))
 (segment (start 167.64 114.14125) (end 180.964779 114.14125) (width 0.2) (layer "F.Cu") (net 7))
 (via (at 180.99221 114.168681) (size 0.6) (drill 0.3) (layers "F.Cu" "B.Cu") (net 7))
 (segment (start 180.99221 113.61721) (end 180.975 113.6) (width 0.2) (layer "B.Cu") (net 7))
 (segment (start 180.99221 114.168681) (end 180.99221 113.61721) (width 0.2) (layer "B.Cu") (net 7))
 (segment (start 186.69 114.14125) (end 200.014779 114.14125) (width 0.2) (layer "F.Cu") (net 4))
 (segment (start 200.014779 114.14125) (end 200.04221 114.168681) (width 0.2) (layer "F.Cu") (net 4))
 (via (at 200.04221 114.168681) (size 0.6) (drill 0.3) (layers "F.Cu" "B.Cu") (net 4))
 (segment (start 200.04221 113.61721) (end 200.025 113.6) (width 0.2) (layer "B.Cu") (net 4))
 (segment (start 200.04221 114.168681) (end 200.04221 113.61721) (width 0.2) (layer "B.Cu") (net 4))
 (segment (start 154.94 73.50125) (end 154.94 92.55125) (width 0.2) (layer "F.Cu") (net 5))
 (segment (start 163.83 64.77) (end 155.09875 73.50125) (width 0.2) (layer "F.Cu") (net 5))
 (segment (start 155.09875 73.50125) (end 154.94 73.50125) (width 0.2) (layer "F.Cu") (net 5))
 (segment (start 154.94 92.55125) (end 154.94 111.60125) (width 0.2) (layer "F.Cu") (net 5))
 (segment (start 179.07 68.42125) (end 173.99 73.50125) (width 0.2) (layer "F.Cu") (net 1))
 (segment (start 173.99 73.50125) (end 173.99 92.55125) (width 0.2) (layer "F.Cu") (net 1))
 (segment (start 179.07 64.77) (end 179.07 68.42125) (width 0.2) (layer "F.Cu") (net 1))
 (segment (start 173.99 92.55125) (end 173.99 111.60125) (width 0.2) (layer "F.Cu") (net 1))
 (segment (start 181.76875 62.23) (end 193.04 73.50125) (width 0.2) (layer "F.Cu") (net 3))
 (segment (start 193.04 73.50125) (end 193.04 92.55125) (width 0.2) (layer "F.Cu") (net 3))
 (segment (start 179.905 62.23) (end 181.76875 62.23) (width 0.2) (layer "F.Cu") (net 3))
 (segment (start 193.04 92.55125) (end 193.04 111.60125) (width 0.2) (layer "F.Cu") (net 3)))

